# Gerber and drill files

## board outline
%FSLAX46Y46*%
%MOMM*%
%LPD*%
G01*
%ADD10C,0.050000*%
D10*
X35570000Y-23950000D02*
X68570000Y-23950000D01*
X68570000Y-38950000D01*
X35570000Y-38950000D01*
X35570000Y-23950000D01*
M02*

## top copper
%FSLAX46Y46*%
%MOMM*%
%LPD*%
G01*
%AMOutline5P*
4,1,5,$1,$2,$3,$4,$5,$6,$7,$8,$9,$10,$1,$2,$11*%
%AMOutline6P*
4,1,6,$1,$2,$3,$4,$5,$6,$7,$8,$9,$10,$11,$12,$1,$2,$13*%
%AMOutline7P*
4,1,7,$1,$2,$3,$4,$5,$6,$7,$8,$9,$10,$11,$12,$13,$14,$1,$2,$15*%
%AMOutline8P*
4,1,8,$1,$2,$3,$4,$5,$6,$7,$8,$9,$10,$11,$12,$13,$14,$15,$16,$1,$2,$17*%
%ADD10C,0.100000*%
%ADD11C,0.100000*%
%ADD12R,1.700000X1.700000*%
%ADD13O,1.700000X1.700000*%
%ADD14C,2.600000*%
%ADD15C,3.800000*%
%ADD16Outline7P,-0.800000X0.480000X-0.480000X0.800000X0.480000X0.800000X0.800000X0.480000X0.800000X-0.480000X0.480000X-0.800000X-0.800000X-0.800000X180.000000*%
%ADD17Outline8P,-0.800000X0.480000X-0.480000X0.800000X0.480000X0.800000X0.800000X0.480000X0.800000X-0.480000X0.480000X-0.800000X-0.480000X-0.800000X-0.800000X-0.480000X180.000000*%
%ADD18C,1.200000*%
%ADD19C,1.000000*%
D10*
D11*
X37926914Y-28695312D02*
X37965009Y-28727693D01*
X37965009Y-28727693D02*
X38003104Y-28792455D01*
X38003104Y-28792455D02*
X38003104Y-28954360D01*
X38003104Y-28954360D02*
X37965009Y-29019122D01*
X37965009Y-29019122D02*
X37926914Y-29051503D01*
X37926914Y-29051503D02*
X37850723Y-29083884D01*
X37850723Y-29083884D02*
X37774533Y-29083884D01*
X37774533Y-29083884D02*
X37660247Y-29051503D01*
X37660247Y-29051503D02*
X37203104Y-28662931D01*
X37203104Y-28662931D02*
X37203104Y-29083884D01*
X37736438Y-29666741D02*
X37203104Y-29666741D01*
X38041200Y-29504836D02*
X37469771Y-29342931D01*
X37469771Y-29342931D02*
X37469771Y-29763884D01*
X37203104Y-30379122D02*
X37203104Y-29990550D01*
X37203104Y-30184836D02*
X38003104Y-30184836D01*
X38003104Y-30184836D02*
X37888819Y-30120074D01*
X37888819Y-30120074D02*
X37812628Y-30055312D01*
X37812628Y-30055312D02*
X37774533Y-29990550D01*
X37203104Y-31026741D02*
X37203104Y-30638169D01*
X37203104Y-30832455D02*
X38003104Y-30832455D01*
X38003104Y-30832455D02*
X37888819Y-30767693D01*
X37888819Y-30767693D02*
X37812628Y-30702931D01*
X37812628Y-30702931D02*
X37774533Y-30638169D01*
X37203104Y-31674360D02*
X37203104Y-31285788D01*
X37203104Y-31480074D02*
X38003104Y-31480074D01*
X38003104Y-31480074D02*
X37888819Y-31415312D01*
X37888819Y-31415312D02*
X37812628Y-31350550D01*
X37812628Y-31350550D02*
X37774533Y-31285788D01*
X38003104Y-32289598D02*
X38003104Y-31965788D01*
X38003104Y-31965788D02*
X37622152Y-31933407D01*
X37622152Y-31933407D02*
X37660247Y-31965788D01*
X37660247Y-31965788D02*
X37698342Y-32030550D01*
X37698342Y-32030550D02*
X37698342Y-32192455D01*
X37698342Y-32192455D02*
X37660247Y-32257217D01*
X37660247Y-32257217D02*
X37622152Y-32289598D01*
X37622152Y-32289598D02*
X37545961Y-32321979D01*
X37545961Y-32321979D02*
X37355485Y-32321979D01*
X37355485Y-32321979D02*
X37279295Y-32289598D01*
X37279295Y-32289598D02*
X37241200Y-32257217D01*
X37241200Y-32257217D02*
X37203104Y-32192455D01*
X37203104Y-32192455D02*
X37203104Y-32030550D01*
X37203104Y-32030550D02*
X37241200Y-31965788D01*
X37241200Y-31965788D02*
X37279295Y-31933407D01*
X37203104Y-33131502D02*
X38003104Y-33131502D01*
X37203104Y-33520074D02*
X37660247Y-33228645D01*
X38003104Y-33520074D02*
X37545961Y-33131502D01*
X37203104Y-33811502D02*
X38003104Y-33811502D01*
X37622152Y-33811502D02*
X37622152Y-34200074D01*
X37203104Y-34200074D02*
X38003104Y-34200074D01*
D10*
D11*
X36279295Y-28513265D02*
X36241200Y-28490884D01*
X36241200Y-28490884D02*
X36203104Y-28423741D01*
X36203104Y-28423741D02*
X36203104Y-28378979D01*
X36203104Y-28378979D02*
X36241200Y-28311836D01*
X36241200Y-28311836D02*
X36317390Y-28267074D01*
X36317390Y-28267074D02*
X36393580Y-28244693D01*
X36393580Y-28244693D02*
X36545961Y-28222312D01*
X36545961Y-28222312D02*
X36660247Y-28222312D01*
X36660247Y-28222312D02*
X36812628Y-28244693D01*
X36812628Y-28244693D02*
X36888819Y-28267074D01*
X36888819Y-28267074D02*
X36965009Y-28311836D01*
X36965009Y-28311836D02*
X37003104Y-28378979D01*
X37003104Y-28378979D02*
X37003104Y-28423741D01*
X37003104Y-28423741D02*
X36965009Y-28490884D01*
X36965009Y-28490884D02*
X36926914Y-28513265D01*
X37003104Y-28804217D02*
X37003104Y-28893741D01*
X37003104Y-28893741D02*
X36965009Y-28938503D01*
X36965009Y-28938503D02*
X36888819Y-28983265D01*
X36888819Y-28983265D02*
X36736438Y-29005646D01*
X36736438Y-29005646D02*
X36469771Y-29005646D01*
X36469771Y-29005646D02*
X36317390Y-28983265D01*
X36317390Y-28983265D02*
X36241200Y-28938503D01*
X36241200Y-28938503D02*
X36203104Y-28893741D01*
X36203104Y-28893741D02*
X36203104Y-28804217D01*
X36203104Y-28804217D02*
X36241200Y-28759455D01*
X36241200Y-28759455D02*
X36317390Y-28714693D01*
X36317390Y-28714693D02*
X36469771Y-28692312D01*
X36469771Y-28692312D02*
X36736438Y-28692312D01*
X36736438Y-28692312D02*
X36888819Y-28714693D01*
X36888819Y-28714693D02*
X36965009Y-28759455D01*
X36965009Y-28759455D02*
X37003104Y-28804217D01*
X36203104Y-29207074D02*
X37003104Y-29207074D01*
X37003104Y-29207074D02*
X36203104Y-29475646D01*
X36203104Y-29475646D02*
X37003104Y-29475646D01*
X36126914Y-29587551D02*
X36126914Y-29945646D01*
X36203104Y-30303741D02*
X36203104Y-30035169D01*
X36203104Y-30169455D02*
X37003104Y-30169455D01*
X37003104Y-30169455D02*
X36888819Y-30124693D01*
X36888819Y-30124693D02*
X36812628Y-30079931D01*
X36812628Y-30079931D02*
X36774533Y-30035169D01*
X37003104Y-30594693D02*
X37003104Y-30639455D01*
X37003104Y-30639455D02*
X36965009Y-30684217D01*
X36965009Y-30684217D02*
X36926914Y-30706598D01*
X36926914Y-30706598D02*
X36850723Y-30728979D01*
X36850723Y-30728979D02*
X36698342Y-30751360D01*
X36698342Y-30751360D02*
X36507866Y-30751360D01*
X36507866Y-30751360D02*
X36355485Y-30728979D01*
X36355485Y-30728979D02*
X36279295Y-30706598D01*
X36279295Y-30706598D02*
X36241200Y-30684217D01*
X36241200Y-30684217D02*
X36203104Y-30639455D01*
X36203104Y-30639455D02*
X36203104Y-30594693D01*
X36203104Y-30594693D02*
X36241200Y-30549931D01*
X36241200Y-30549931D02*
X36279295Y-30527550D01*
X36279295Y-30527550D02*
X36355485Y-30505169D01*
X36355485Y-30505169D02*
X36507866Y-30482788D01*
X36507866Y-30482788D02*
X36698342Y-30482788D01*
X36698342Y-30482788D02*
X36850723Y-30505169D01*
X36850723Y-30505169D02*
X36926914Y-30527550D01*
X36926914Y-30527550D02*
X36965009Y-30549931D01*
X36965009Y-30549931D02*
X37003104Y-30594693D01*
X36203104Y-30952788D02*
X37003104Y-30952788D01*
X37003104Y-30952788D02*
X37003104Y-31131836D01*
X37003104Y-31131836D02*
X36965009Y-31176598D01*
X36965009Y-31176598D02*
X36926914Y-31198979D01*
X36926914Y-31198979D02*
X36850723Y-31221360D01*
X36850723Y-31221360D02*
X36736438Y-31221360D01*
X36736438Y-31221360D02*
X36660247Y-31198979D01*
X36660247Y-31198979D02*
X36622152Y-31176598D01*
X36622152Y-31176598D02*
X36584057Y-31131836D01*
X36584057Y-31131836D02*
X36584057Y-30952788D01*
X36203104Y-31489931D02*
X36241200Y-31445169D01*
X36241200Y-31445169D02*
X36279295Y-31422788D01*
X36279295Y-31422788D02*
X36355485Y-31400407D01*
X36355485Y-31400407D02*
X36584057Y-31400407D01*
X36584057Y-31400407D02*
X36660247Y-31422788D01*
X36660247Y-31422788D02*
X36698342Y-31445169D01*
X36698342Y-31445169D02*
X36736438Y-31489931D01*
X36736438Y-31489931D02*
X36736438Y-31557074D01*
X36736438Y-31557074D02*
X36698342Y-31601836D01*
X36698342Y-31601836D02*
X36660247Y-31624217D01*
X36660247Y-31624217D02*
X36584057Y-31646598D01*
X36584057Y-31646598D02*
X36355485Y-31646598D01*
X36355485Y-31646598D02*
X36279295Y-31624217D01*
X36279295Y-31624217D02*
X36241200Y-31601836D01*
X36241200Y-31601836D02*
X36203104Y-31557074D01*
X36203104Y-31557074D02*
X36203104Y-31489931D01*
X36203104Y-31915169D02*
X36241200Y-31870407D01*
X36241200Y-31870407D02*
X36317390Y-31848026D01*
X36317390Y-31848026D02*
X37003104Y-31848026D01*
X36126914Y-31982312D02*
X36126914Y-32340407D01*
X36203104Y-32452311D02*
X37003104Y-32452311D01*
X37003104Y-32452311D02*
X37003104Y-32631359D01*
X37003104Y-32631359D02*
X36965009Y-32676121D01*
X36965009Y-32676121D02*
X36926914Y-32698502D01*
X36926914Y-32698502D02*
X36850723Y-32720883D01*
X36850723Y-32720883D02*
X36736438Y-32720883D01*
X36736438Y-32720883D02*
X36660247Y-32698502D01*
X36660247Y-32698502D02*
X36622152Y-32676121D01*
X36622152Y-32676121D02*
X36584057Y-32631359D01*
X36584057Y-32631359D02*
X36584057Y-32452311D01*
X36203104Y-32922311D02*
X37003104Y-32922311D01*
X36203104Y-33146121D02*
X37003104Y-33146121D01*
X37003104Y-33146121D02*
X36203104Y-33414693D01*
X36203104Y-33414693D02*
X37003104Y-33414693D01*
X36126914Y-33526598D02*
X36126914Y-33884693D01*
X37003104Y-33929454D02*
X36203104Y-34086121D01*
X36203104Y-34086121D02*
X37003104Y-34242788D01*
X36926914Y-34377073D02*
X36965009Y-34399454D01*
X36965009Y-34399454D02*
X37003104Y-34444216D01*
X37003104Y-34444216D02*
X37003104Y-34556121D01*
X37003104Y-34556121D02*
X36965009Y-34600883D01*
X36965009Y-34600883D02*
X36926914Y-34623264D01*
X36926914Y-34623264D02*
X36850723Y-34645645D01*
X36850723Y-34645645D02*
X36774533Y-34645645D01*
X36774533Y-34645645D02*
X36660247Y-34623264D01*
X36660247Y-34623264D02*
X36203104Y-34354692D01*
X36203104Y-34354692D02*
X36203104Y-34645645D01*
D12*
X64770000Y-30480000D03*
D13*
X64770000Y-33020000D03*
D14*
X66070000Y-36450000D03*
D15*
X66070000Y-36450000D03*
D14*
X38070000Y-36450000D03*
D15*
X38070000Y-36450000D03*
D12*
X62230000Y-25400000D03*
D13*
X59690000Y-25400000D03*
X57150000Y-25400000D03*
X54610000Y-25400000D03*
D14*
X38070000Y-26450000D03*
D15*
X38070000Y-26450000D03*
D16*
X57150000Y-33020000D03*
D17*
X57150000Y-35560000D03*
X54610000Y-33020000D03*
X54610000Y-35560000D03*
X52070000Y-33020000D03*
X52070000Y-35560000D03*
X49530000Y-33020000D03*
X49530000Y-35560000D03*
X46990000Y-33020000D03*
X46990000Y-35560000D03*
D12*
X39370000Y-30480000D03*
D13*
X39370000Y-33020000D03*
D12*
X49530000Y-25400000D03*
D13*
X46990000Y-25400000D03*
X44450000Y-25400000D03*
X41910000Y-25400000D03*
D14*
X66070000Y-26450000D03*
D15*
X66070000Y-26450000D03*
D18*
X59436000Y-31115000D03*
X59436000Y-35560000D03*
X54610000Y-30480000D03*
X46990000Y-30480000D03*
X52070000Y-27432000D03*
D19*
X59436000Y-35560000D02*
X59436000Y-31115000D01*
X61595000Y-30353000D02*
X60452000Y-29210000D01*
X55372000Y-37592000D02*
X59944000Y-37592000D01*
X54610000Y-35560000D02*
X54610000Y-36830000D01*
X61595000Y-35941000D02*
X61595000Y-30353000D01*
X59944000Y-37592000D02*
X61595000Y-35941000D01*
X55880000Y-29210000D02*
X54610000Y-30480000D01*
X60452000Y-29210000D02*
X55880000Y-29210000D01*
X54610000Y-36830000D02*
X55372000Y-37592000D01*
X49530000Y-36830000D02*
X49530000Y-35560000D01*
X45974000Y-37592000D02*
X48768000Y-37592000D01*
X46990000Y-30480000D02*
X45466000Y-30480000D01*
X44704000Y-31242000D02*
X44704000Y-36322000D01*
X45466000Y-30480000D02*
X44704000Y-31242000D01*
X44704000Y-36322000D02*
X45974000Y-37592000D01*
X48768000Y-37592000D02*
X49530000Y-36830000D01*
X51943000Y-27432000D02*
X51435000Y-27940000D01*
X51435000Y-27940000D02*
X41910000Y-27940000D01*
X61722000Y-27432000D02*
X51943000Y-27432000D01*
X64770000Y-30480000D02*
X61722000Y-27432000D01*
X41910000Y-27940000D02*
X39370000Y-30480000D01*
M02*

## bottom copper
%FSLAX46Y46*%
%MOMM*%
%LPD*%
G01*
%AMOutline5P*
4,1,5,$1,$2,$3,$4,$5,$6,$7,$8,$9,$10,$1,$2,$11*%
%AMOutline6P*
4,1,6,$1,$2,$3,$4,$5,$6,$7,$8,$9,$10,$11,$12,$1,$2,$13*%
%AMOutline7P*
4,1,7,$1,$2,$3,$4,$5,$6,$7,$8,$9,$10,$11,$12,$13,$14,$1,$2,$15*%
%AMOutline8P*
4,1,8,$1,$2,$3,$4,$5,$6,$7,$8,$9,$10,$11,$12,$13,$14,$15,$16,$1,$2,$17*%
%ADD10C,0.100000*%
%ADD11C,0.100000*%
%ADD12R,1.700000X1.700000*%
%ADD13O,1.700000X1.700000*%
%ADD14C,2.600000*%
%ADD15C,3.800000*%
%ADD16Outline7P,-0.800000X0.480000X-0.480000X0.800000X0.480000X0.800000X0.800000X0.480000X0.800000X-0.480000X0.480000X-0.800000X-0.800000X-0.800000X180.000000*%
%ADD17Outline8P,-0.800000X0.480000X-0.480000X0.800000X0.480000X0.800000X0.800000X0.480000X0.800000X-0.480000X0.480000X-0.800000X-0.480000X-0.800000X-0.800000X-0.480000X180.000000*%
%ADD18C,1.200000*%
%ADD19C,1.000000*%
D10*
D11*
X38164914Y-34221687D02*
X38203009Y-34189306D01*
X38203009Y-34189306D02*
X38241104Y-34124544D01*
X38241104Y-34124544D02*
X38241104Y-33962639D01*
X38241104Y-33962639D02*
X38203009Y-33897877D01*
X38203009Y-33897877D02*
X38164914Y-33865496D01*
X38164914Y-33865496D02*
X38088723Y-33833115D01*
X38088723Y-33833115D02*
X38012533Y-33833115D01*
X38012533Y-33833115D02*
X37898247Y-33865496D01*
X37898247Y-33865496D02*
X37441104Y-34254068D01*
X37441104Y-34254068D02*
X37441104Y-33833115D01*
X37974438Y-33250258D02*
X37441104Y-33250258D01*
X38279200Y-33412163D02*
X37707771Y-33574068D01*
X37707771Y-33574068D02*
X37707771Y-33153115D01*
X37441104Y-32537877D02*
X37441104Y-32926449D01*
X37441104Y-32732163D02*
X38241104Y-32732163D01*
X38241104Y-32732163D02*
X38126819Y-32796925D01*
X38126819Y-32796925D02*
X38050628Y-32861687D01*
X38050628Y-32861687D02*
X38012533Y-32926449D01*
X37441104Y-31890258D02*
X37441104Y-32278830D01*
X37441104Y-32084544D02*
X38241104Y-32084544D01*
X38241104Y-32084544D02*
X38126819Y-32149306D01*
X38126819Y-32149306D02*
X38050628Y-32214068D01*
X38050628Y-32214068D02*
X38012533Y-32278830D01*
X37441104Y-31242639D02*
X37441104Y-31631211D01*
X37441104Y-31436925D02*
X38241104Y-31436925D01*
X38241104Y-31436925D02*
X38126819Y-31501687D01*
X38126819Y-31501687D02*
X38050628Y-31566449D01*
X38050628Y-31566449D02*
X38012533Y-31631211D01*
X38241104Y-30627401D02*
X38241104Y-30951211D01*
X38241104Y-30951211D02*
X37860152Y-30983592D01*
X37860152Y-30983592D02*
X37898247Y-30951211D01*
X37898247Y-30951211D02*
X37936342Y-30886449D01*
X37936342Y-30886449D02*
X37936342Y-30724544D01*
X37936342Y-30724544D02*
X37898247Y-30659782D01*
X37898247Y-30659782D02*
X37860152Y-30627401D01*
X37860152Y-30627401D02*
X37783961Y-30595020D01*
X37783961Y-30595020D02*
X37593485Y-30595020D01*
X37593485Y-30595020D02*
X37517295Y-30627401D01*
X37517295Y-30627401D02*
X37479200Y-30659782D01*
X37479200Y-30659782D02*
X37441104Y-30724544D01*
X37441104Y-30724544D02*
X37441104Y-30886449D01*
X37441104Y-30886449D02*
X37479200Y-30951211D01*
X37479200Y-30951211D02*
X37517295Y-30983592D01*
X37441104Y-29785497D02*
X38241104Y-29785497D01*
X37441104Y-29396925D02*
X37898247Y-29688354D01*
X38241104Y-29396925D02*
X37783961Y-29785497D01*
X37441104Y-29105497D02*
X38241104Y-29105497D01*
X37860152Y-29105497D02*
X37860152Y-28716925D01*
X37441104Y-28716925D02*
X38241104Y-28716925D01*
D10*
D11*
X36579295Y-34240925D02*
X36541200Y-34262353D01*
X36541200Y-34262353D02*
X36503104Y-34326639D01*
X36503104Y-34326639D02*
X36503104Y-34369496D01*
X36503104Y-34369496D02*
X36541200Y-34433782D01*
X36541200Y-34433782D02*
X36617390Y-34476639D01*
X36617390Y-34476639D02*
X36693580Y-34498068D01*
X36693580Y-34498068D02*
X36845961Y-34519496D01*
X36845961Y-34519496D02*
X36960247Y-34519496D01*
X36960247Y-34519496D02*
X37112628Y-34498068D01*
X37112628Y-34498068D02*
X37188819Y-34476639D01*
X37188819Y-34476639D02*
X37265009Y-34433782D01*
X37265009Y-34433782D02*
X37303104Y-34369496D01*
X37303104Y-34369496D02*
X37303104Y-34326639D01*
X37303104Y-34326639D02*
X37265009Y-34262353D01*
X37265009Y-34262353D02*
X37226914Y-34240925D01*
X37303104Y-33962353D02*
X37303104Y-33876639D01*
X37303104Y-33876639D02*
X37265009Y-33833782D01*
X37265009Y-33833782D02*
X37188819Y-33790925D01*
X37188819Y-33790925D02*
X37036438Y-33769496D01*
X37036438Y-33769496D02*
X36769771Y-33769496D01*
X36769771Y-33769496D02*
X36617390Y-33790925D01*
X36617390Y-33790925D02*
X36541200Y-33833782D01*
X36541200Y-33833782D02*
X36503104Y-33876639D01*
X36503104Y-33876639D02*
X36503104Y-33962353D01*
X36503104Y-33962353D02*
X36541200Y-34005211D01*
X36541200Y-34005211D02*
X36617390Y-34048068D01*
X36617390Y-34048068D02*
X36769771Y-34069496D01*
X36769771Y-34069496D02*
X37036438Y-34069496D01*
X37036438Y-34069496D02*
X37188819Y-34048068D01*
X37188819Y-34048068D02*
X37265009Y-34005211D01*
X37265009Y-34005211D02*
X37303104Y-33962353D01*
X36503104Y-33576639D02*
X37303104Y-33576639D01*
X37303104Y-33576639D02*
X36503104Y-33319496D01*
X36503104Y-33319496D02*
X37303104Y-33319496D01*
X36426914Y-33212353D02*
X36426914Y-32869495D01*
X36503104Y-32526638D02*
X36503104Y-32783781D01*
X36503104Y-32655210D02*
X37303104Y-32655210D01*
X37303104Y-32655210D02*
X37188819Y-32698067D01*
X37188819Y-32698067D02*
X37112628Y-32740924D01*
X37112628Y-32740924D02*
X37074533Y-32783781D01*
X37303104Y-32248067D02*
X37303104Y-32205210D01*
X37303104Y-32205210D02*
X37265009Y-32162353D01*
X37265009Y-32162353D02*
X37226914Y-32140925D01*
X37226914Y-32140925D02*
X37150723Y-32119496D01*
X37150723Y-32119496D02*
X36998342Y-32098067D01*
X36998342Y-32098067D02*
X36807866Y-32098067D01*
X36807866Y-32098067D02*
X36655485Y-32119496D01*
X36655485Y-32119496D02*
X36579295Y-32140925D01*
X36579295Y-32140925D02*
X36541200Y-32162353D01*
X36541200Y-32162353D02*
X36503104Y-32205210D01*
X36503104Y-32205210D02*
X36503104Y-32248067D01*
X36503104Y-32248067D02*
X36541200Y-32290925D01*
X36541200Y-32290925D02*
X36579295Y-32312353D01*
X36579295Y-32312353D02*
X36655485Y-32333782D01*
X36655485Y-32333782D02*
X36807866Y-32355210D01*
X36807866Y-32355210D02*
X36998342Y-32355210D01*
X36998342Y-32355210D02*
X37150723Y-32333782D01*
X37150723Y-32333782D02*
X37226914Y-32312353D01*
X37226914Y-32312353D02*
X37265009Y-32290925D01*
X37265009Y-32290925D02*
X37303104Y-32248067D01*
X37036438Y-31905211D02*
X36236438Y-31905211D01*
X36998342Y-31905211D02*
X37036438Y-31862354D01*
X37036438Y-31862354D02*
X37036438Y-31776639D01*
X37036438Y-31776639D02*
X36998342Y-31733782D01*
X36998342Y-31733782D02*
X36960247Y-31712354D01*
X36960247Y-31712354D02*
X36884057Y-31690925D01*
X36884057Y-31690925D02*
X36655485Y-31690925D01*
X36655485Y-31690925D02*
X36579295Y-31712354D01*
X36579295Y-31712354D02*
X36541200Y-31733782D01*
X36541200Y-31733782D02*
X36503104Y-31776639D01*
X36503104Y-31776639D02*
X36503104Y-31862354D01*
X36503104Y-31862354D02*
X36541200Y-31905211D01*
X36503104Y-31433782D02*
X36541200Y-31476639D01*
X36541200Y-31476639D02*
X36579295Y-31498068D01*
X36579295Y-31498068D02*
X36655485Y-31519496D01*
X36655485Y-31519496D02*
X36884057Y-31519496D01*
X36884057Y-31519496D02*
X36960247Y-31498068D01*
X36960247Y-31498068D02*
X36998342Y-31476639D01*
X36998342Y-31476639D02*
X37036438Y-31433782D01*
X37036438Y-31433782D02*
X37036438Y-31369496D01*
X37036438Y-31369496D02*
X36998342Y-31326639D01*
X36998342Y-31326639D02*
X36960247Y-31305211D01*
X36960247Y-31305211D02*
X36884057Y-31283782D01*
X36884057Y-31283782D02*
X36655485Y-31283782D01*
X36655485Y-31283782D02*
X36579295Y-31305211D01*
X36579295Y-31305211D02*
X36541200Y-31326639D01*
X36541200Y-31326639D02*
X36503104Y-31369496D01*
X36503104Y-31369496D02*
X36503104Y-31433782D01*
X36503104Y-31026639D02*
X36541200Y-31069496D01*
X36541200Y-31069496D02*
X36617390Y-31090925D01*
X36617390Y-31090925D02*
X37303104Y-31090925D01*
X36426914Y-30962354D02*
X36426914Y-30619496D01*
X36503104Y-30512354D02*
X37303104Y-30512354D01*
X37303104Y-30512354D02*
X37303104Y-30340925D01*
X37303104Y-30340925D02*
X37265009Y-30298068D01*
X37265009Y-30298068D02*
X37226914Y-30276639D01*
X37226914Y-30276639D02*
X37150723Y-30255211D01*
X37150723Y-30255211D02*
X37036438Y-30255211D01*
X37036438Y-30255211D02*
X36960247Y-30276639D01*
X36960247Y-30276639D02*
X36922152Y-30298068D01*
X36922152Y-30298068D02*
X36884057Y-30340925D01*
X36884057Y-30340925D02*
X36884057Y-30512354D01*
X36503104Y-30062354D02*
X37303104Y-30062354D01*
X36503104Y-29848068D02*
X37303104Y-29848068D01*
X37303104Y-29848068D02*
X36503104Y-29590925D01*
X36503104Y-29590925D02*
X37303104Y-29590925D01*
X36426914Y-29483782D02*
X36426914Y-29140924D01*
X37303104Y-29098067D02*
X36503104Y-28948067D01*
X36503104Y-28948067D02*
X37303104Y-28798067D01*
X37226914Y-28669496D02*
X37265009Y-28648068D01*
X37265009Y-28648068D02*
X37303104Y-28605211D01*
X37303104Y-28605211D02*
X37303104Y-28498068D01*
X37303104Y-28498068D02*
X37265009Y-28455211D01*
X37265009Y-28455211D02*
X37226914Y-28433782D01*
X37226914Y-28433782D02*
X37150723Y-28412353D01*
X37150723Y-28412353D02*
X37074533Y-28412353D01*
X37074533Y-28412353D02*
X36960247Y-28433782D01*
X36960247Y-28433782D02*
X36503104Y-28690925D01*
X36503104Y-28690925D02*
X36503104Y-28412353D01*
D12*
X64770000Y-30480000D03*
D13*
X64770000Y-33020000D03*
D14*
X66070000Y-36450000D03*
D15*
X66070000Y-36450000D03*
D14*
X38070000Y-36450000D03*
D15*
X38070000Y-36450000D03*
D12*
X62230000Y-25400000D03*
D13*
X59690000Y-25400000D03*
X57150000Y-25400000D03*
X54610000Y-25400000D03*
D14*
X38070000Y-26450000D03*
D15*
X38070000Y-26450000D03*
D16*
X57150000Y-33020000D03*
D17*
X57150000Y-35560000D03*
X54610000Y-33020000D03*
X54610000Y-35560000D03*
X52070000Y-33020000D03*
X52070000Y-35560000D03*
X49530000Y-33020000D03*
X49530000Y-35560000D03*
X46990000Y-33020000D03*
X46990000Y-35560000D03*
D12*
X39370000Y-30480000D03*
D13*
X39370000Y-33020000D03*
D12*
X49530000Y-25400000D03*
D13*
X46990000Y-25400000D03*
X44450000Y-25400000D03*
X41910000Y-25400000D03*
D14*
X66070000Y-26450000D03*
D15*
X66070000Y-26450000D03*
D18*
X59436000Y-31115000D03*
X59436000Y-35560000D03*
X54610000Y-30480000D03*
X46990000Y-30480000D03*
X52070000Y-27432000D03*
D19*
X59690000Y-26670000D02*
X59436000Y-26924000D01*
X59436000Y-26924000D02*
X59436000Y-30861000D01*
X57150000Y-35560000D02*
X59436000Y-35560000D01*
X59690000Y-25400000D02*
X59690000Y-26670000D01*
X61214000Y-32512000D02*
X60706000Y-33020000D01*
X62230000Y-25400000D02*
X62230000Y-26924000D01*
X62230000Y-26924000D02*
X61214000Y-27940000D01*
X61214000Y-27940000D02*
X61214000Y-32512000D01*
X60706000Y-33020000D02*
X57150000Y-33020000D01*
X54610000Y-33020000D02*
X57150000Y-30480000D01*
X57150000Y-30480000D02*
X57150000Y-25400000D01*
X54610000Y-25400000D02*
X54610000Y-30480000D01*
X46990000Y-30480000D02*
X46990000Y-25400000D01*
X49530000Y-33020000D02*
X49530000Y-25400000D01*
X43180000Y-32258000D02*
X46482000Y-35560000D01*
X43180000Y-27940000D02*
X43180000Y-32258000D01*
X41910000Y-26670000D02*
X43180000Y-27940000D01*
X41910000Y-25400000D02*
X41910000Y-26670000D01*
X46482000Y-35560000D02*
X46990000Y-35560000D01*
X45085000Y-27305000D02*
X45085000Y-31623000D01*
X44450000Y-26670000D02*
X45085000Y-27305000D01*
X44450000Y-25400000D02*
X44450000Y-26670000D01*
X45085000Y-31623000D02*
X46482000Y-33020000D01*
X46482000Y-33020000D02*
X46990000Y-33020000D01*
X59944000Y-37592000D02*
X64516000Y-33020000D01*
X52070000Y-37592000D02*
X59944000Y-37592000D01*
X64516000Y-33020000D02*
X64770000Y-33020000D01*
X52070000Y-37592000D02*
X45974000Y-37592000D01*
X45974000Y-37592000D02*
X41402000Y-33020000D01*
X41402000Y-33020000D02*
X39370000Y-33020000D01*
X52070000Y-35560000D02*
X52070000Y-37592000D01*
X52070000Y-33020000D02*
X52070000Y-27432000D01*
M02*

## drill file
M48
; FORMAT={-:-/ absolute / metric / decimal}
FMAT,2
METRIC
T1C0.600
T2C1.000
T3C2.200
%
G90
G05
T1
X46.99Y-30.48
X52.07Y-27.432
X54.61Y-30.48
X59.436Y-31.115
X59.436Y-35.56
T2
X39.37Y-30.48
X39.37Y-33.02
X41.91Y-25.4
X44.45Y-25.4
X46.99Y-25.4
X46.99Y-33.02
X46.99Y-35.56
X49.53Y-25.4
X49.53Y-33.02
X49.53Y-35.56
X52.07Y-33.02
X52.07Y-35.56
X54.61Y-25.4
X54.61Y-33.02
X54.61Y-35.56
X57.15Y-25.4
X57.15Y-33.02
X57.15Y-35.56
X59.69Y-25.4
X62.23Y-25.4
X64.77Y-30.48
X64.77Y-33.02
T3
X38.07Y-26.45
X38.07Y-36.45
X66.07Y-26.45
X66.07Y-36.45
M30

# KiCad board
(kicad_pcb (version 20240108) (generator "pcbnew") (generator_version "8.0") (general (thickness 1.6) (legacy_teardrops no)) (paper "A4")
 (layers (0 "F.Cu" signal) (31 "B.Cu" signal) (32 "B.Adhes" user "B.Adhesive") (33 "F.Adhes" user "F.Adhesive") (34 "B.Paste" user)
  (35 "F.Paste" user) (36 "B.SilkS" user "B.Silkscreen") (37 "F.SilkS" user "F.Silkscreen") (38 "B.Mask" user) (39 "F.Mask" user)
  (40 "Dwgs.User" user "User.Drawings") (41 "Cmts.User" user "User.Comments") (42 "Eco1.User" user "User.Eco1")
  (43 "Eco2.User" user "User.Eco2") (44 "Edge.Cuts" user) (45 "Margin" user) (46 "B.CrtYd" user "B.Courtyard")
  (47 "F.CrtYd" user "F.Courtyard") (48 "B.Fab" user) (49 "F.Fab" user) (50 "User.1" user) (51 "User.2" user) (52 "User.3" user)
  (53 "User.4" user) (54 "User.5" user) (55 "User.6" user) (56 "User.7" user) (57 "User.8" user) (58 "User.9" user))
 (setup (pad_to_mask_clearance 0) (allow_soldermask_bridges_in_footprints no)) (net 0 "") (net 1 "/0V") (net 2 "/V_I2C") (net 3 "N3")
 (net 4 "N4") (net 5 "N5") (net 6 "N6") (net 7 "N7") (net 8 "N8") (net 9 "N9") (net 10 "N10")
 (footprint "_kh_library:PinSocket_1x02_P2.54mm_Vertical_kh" (layer "F.Cu") (at 64.77 30.48)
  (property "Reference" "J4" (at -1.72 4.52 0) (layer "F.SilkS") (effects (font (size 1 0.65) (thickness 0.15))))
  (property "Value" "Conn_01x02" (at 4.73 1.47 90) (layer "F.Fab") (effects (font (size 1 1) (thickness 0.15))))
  (pad "1" thru_hole rect (at 0 0) (size 1.7 1.7) (drill 1) (layers "*.Cu" "*.Mask") (remove_unused_layers no) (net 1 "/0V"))
  (pad "2" thru_hole oval (at 0 2.54) (size 1.7 1.7) (drill 1) (layers "*.Cu" "*.Mask") (remove_unused_layers no) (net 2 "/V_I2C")))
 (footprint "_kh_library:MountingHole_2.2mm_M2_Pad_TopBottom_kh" (layer "F.Cu") (at 66.07 36.45)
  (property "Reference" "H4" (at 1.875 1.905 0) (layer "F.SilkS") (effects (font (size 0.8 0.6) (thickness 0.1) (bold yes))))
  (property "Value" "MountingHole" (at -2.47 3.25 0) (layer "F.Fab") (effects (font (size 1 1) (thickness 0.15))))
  (pad "1" thru_hole circle (at 0 0) (size 2.6 2.6) (drill 2.2) (layers "*.Cu" "*.Mask") (remove_unused_layers no))
  (pad "1" connect circle (at 0 0) (size 3.8 3.8) (layers "F.Cu" "F.Mask"))
  (pad "1" connect circle (at 0 0) (size 3.8 3.8) (layers "B.Cu" "B.Mask")))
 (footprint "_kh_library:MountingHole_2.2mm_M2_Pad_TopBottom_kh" (layer "F.Cu") (at 38.07 36.45)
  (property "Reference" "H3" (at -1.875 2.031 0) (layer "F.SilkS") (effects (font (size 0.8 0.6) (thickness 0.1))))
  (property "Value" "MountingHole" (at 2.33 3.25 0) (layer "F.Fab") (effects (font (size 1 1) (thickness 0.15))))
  (pad "1" thru_hole circle (at 0 0) (size 2.6 2.6) (drill 2.2) (layers "*.Cu" "*.Mask") (remove_unused_layers no))
  (pad "1" connect circle (at 0 0) (size 3.8 3.8) (layers "F.Cu" "F.Mask"))
  (pad "1" connect circle (at 0 0) (size 3.8 3.8) (layers "B.Cu" "B.Mask")))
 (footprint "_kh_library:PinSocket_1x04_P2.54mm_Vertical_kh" (layer "F.Cu") (at 62.23 25.4 -90)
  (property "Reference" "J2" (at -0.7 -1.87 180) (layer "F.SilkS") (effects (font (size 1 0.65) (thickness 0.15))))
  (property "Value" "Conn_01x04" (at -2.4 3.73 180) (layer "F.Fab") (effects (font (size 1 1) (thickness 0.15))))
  (pad "1" thru_hole rect (at 0 0 270) (size 1.7 1.7) (drill 1) (layers "*.Cu" "*.Mask") (remove_unused_layers no) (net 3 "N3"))
  (pad "2" thru_hole oval (at 0 2.54 270) (size 1.7 1.7) (drill 1) (layers "*.Cu" "*.Mask") (remove_unused_layers no) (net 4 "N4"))
  (pad "3" thru_hole oval (at 0 5.08 270) (size 1.7 1.7) (drill 1) (layers "*.Cu" "*.Mask") (remove_unused_layers no) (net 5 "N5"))
  (pad "4" thru_hole oval (at 0 7.62 270) (size 1.7 1.7) (drill 1) (layers "*.Cu" "*.Mask") (remove_unused_layers no) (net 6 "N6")))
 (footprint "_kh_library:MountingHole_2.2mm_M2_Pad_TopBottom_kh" (layer "F.Cu") (at 38.07 26.45)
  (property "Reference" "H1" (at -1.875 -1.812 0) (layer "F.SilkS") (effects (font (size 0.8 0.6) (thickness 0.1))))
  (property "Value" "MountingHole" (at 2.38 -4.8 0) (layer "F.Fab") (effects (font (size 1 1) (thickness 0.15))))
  (pad "1" thru_hole circle (at 0 0) (size 2.6 2.6) (drill 2.2) (layers "*.Cu" "*.Mask") (remove_unused_layers no))
  (pad "1" connect circle (at 0 0) (size 3.8 3.8) (layers "F.Cu" "F.Mask"))
  (pad "1" connect circle (at 0 0) (size 3.8 3.8) (layers "B.Cu" "B.Mask")))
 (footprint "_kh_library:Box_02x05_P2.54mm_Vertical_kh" (layer "F.Cu") (at 57.15 33.02 180)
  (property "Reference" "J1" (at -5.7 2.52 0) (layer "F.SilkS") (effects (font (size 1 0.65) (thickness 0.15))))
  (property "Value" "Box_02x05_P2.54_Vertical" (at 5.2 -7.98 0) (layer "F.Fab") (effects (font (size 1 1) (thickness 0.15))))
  (pad "1" thru_hole roundrect (at 0 0 180) (size 1.6 1.6) (drill 1) (layers "*.Cu" "*.Mask") (remove_unused_layers no) (roundrect_rratio 0)
   (chamfer_ratio 0.2) (chamfer top_left top_right bottom_right) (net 3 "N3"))
  (pad "2" thru_hole roundrect (at 0 -2.54 180) (size 1.6 1.6) (drill 1) (layers "*.Cu" "*.Mask") (remove_unused_layers no)
   (roundrect_rratio 0) (chamfer_ratio 0.2) (chamfer top_left top_right bottom_left bottom_right) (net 4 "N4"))
  (pad "3" thru_hole roundrect (at 2.54 0 180) (size 1.6 1.6) (drill 1) (layers "*.Cu" "*.Mask") (remove_unused_layers no)
   (roundrect_rratio 0) (chamfer_ratio 0.2) (chamfer top_left top_right bottom_left bottom_right) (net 5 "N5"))
  (pad "4" thru_hole roundrect (at 2.54 -2.54 180) (size 1.6 1.6) (drill 1) (layers "*.Cu" "*.Mask") (remove_unused_layers no)
   (roundrect_rratio 0) (chamfer_ratio 0.2) (chamfer top_left top_right bottom_left bottom_right) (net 6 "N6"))
  (pad "5" thru_hole roundrect (at 5.08 0 180) (size 1.6 1.6) (drill 1) (layers "*.Cu" "*.Mask") (remove_unused_layers no)
   (roundrect_rratio 0) (chamfer_ratio 0.2) (chamfer top_left top_right bottom_left bottom_right) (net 1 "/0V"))
  (pad "6" thru_hole roundrect (at 5.08 -2.54 180) (size 1.6 1.6) (drill 1) (layers "*.Cu" "*.Mask") (remove_unused_layers no)
   (roundrect_rratio 0) (chamfer_ratio 0.2) (chamfer top_left top_right bottom_left bottom_right) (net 2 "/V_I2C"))
  (pad "7" thru_hole roundrect (at 7.62 0 180) (size 1.6 1.6) (drill 1) (layers "*.Cu" "*.Mask") (remove_unused_layers no)
   (roundrect_rratio 0) (chamfer_ratio 0.2) (chamfer top_left top_right bottom_left bottom_right) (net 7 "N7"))
  (pad "8" thru_hole roundrect (at 7.62 -2.54 180) (size 1.6 1.6) (drill 1) (layers "*.Cu" "*.Mask") (remove_unused_layers no)
   (roundrect_rratio 0) (chamfer_ratio 0.2) (chamfer top_left top_right bottom_left bottom_right) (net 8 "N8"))
  (pad "9" thru_hole roundrect (at 10.16 0 180) (size 1.6 1.6) (drill 1) (layers "*.Cu" "*.Mask") (remove_unused_layers no)
   (roundrect_rratio 0) (chamfer_ratio 0.2) (chamfer top_left top_right bottom_left bottom_right) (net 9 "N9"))
  (pad "10" thru_hole roundrect (at 10.16 -2.54 180) (size 1.6 1.6) (drill 1) (layers "*.Cu" "*.Mask") (remove_unused_layers no)
   (roundrect_rratio 0) (chamfer_ratio 0.2) (chamfer top_left top_right bottom_left bottom_right) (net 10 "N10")))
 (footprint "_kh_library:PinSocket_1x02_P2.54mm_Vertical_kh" (layer "F.Cu") (at 39.37 30.48)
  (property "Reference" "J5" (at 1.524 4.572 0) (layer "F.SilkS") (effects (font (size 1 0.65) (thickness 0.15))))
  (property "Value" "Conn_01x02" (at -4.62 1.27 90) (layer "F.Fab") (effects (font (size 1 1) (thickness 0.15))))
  (pad "1" thru_hole rect (at 0 0) (size 1.7 1.7) (drill 1) (layers "*.Cu" "*.Mask") (remove_unused_layers no) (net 1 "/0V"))
  (pad "2" thru_hole oval (at 0 2.54) (size 1.7 1.7) (drill 1) (layers "*.Cu" "*.Mask") (remove_unused_layers no) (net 2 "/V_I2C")))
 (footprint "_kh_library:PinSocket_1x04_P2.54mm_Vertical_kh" (layer "F.Cu") (at 49.53 25.4 -90)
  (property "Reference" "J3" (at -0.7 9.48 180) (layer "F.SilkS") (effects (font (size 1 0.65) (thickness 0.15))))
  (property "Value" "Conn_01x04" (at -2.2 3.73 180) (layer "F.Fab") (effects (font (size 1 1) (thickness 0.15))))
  (pad "1" thru_hole rect (at 0 0 270) (size 1.7 1.7) (drill 1) (layers "*.Cu" "*.Mask") (remove_unused_layers no) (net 7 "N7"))
  (pad "2" thru_hole oval (at 0 2.54 270) (size 1.7 1.7) (drill 1) (layers "*.Cu" "*.Mask") (remove_unused_layers no) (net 8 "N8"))
  (pad "3" thru_hole oval (at 0 5.08 270) (size 1.7 1.7) (drill 1) (layers "*.Cu" "*.Mask") (remove_unused_layers no) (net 9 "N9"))
  (pad "4" thru_hole oval (at 0 7.62 270) (size 1.7 1.7) (drill 1) (layers "*.Cu" "*.Mask") (remove_unused_layers no) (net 10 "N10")))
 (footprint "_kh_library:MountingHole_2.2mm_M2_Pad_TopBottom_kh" (layer "F.Cu") (at 66.07 26.45)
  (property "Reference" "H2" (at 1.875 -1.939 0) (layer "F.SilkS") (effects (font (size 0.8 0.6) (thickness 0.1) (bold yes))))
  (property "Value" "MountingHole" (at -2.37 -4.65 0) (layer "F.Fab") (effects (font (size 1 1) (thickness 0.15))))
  (pad "1" thru_hole circle (at 0 0) (size 2.6 2.6) (drill 2.2) (layers "*.Cu" "*.Mask") (remove_unused_layers no))
  (pad "1" connect circle (at 0 0) (size 3.8 3.8) (layers "F.Cu" "F.Mask"))
  (pad "1" connect circle (at 0 0) (size 3.8 3.8) (layers "B.Cu" "B.Mask")))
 (gr_rect (start 35.57 23.95) (end 68.57 38.95) (stroke (width 0.05) (type default)) (fill none) (layer "Edge.Cuts"))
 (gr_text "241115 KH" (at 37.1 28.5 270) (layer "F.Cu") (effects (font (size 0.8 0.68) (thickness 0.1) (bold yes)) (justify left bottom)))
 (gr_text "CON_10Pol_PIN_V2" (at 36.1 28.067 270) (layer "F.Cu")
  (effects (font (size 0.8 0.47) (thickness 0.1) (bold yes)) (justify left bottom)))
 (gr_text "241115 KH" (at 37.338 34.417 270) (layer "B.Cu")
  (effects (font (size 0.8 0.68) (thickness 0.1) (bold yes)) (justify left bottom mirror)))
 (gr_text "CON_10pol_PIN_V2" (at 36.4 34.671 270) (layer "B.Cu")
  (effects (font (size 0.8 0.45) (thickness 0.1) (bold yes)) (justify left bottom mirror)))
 (segment (start 59.436 35.56) (end 59.436 31.115) (width 1) (layer "F.Cu") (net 4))
 (via (at 59.436 31.115) (size 1.2) (drill 0.6) (layers "F.Cu" "B.Cu") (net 4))
 (via (at 59.436 35.56) (size 1.2) (drill 0.6) (layers "F.Cu" "B.Cu") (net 4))
 (segment (start 59.69 26.67) (end 59.436 26.924) (width 1) (layer "B.Cu") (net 4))
 (segment (start 59.436 26.924) (end 59.436 30.861) (width 1) (layer "B.Cu") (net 4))
 (segment (start 57.15 35.56) (end 59.436 35.56) (width 1) (layer "B.Cu") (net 4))
 (segment (start 59.69 25.4) (end 59.69 26.67) (width 1) (layer "B.Cu") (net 4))
 (segment (start 61.214 32.512) (end 60.706 33.02) (width 1) (layer "B.Cu") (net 3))
 (segment (start 62.23 25.4) (end 62.23 26.924) (width 1) (layer "B.Cu") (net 3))
 (segment (start 62.23 26.924) (end 61.214 27.94) (width 1) (layer "B.Cu") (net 3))
 (segment (start 61.214 27.94) (end 61.214 32.512) (width 1) (layer "B.Cu") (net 3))
 (segment (start 60.706 33.02) (end 57.15 33.02) (width 1) (layer "B.Cu") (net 3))
 (segment (start 54.61 33.02) (end 57.15 30.48) (width 1) (layer "B.Cu") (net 5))
 (segment (start 57.15 30.48) (end 57.15 25.4) (width 1) (layer "B.Cu") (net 5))
 (segment (start 61.595 30.353) (end 60.452 29.21) (width 1) (layer "F.Cu") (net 6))
 (segment (start 55.372 37.592) (end 59.944 37.592) (width 1) (layer "F.Cu") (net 6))
 (segment (start 54.61 35.56) (end 54.61 36.83) (width 1) (layer "F.Cu") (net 6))
 (segment (start 61.595 35.941) (end 61.595 30.353) (width 1) (layer "F.Cu") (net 6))
 (segment (start 59.944 37.592) (end 61.595 35.941) (width 1) (layer "F.Cu") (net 6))
 (segment (start 55.88 29.21) (end 54.61 30.48) (width 1) (layer "F.Cu") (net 6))
 (segment (start 60.452 29.21) (end 55.88 29.21) (width 1) (layer "F.Cu") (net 6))
 (segment (start 54.61 36.83) (end 55.372 37.592) (width 1) (layer "F.Cu") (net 6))
 (via (at 54.61 30.48) (size 1.2) (drill 0.6) (layers "F.Cu" "B.Cu") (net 6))
 (segment (start 54.61 25.4) (end 54.61 30.48) (width 1) (layer "B.Cu") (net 6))
 (segment (start 49.53 36.83) (end 49.53 35.56) (width 1) (layer "F.Cu") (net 8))
 (segment (start 45.974 37.592) (end 48.768 37.592) (width 1) (layer "F.Cu") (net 8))
 (segment (start 46.99 30.48) (end 45.466 30.48) (width 1) (layer "F.Cu") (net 8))
 (segment (start 44.704 31.242) (end 44.704 36.322) (width 1) (layer "F.Cu") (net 8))
 (segment (start 45.466 30.48) (end 44.704 31.242) (width 1) (layer "F.Cu") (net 8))
 (segment (start 44.704 36.322) (end 45.974 37.592) (width 1) (layer "F.Cu") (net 8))
 (segment (start 48.768 37.592) (end 49.53 36.83) (width 1) (layer "F.Cu") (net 8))
 (via (at 46.99 30.48) (size 1.2) (drill 0.6) (layers "F.Cu" "B.Cu") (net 8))
 (segment (start 46.99 30.48) (end 46.99 25.4) (width 1) (layer "B.Cu") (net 8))
 (segment (start 49.53 33.02) (end 49.53 25.4) (width 1) (layer "B.Cu") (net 7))
 (segment (start 43.18 32.258) (end 46.482 35.56) (width 1) (layer "B.Cu") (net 10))
 (segment (start 43.18 27.94) (end 43.18 32.258) (width 1) (layer "B.Cu") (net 10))
 (segment (start 41.91 26.67) (end 43.18 27.94) (width 1) (layer "B.Cu") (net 10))
 (segment (start 41.91 25.4) (end 41.91 26.67) (width 1) (layer "B.Cu") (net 10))
 (segment (start 46.482 35.56) (end 46.99 35.56) (width 1) (layer "B.Cu") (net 10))
 (segment (start 45.085 27.305) (end 45.085 31.623) (width 1) (layer "B.Cu") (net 9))
 (segment (start 44.45 26.67) (end 45.085 27.305) (width 1) (layer "B.Cu") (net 9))
 (segment (start 44.45 25.4) (end 44.45 26.67) (width 1) (layer "B.Cu") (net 9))
 (segment (start 45.085 31.623) (end 46.482 33.02) (width 1) (layer "B.Cu") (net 9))
 (segment (start 46.482 33.02) (end 46.99 33.02) (width 1) (layer "B.Cu") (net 9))
 (segment (start 59.944 37.592) (end 64.516 33.02) (width 1) (layer "B.Cu") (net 2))
 (segment (start 52.07 37.592) (end 59.944 37.592) (width 1) (layer "B.Cu") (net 2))
 (segment (start 64.516 33.02) (end 64.77 33.02) (width 1) (layer "B.Cu") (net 2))
 (segment (start 52.07 37.592) (end 45.974 37.592) (width 1) (layer "B.Cu") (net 2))
 (segment (start 45.974 37.592) (end 41.402 33.02) (width 1) (layer "B.Cu") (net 2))
 (segment (start 41.402 33.02) (end 39.37 33.02) (width 1) (layer "B.Cu") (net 2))
 (segment (start 52.07 35.56) (end 52.07 37.592) (width 1) (layer "B.Cu") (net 2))
 (segment (start 51.943 27.432) (end 51.435 27.94) (width 1) (layer "F.Cu") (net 1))
 (segment (start 51.435 27.94) (end 41.91 27.94) (width 1) (layer "F.Cu") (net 1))
 (segment (start 61.722 27.432) (end 51.943 27.432) (width 1) (layer "F.Cu") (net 1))
 (segment (start 64.77 30.48) (end 61.722 27.432) (width 1) (layer "F.Cu") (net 1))
 (segment (start 41.91 27.94) (end 39.37 30.48) (width 1) (layer "F.Cu") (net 1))
 (via (at 52.07 27.432) (size 1.2) (drill 0.6) (layers "F.Cu" "B.Cu") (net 1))
 (segment (start 52.07 33.02) (end 52.07 27.432) (width 1) (layer "B.Cu") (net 1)))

